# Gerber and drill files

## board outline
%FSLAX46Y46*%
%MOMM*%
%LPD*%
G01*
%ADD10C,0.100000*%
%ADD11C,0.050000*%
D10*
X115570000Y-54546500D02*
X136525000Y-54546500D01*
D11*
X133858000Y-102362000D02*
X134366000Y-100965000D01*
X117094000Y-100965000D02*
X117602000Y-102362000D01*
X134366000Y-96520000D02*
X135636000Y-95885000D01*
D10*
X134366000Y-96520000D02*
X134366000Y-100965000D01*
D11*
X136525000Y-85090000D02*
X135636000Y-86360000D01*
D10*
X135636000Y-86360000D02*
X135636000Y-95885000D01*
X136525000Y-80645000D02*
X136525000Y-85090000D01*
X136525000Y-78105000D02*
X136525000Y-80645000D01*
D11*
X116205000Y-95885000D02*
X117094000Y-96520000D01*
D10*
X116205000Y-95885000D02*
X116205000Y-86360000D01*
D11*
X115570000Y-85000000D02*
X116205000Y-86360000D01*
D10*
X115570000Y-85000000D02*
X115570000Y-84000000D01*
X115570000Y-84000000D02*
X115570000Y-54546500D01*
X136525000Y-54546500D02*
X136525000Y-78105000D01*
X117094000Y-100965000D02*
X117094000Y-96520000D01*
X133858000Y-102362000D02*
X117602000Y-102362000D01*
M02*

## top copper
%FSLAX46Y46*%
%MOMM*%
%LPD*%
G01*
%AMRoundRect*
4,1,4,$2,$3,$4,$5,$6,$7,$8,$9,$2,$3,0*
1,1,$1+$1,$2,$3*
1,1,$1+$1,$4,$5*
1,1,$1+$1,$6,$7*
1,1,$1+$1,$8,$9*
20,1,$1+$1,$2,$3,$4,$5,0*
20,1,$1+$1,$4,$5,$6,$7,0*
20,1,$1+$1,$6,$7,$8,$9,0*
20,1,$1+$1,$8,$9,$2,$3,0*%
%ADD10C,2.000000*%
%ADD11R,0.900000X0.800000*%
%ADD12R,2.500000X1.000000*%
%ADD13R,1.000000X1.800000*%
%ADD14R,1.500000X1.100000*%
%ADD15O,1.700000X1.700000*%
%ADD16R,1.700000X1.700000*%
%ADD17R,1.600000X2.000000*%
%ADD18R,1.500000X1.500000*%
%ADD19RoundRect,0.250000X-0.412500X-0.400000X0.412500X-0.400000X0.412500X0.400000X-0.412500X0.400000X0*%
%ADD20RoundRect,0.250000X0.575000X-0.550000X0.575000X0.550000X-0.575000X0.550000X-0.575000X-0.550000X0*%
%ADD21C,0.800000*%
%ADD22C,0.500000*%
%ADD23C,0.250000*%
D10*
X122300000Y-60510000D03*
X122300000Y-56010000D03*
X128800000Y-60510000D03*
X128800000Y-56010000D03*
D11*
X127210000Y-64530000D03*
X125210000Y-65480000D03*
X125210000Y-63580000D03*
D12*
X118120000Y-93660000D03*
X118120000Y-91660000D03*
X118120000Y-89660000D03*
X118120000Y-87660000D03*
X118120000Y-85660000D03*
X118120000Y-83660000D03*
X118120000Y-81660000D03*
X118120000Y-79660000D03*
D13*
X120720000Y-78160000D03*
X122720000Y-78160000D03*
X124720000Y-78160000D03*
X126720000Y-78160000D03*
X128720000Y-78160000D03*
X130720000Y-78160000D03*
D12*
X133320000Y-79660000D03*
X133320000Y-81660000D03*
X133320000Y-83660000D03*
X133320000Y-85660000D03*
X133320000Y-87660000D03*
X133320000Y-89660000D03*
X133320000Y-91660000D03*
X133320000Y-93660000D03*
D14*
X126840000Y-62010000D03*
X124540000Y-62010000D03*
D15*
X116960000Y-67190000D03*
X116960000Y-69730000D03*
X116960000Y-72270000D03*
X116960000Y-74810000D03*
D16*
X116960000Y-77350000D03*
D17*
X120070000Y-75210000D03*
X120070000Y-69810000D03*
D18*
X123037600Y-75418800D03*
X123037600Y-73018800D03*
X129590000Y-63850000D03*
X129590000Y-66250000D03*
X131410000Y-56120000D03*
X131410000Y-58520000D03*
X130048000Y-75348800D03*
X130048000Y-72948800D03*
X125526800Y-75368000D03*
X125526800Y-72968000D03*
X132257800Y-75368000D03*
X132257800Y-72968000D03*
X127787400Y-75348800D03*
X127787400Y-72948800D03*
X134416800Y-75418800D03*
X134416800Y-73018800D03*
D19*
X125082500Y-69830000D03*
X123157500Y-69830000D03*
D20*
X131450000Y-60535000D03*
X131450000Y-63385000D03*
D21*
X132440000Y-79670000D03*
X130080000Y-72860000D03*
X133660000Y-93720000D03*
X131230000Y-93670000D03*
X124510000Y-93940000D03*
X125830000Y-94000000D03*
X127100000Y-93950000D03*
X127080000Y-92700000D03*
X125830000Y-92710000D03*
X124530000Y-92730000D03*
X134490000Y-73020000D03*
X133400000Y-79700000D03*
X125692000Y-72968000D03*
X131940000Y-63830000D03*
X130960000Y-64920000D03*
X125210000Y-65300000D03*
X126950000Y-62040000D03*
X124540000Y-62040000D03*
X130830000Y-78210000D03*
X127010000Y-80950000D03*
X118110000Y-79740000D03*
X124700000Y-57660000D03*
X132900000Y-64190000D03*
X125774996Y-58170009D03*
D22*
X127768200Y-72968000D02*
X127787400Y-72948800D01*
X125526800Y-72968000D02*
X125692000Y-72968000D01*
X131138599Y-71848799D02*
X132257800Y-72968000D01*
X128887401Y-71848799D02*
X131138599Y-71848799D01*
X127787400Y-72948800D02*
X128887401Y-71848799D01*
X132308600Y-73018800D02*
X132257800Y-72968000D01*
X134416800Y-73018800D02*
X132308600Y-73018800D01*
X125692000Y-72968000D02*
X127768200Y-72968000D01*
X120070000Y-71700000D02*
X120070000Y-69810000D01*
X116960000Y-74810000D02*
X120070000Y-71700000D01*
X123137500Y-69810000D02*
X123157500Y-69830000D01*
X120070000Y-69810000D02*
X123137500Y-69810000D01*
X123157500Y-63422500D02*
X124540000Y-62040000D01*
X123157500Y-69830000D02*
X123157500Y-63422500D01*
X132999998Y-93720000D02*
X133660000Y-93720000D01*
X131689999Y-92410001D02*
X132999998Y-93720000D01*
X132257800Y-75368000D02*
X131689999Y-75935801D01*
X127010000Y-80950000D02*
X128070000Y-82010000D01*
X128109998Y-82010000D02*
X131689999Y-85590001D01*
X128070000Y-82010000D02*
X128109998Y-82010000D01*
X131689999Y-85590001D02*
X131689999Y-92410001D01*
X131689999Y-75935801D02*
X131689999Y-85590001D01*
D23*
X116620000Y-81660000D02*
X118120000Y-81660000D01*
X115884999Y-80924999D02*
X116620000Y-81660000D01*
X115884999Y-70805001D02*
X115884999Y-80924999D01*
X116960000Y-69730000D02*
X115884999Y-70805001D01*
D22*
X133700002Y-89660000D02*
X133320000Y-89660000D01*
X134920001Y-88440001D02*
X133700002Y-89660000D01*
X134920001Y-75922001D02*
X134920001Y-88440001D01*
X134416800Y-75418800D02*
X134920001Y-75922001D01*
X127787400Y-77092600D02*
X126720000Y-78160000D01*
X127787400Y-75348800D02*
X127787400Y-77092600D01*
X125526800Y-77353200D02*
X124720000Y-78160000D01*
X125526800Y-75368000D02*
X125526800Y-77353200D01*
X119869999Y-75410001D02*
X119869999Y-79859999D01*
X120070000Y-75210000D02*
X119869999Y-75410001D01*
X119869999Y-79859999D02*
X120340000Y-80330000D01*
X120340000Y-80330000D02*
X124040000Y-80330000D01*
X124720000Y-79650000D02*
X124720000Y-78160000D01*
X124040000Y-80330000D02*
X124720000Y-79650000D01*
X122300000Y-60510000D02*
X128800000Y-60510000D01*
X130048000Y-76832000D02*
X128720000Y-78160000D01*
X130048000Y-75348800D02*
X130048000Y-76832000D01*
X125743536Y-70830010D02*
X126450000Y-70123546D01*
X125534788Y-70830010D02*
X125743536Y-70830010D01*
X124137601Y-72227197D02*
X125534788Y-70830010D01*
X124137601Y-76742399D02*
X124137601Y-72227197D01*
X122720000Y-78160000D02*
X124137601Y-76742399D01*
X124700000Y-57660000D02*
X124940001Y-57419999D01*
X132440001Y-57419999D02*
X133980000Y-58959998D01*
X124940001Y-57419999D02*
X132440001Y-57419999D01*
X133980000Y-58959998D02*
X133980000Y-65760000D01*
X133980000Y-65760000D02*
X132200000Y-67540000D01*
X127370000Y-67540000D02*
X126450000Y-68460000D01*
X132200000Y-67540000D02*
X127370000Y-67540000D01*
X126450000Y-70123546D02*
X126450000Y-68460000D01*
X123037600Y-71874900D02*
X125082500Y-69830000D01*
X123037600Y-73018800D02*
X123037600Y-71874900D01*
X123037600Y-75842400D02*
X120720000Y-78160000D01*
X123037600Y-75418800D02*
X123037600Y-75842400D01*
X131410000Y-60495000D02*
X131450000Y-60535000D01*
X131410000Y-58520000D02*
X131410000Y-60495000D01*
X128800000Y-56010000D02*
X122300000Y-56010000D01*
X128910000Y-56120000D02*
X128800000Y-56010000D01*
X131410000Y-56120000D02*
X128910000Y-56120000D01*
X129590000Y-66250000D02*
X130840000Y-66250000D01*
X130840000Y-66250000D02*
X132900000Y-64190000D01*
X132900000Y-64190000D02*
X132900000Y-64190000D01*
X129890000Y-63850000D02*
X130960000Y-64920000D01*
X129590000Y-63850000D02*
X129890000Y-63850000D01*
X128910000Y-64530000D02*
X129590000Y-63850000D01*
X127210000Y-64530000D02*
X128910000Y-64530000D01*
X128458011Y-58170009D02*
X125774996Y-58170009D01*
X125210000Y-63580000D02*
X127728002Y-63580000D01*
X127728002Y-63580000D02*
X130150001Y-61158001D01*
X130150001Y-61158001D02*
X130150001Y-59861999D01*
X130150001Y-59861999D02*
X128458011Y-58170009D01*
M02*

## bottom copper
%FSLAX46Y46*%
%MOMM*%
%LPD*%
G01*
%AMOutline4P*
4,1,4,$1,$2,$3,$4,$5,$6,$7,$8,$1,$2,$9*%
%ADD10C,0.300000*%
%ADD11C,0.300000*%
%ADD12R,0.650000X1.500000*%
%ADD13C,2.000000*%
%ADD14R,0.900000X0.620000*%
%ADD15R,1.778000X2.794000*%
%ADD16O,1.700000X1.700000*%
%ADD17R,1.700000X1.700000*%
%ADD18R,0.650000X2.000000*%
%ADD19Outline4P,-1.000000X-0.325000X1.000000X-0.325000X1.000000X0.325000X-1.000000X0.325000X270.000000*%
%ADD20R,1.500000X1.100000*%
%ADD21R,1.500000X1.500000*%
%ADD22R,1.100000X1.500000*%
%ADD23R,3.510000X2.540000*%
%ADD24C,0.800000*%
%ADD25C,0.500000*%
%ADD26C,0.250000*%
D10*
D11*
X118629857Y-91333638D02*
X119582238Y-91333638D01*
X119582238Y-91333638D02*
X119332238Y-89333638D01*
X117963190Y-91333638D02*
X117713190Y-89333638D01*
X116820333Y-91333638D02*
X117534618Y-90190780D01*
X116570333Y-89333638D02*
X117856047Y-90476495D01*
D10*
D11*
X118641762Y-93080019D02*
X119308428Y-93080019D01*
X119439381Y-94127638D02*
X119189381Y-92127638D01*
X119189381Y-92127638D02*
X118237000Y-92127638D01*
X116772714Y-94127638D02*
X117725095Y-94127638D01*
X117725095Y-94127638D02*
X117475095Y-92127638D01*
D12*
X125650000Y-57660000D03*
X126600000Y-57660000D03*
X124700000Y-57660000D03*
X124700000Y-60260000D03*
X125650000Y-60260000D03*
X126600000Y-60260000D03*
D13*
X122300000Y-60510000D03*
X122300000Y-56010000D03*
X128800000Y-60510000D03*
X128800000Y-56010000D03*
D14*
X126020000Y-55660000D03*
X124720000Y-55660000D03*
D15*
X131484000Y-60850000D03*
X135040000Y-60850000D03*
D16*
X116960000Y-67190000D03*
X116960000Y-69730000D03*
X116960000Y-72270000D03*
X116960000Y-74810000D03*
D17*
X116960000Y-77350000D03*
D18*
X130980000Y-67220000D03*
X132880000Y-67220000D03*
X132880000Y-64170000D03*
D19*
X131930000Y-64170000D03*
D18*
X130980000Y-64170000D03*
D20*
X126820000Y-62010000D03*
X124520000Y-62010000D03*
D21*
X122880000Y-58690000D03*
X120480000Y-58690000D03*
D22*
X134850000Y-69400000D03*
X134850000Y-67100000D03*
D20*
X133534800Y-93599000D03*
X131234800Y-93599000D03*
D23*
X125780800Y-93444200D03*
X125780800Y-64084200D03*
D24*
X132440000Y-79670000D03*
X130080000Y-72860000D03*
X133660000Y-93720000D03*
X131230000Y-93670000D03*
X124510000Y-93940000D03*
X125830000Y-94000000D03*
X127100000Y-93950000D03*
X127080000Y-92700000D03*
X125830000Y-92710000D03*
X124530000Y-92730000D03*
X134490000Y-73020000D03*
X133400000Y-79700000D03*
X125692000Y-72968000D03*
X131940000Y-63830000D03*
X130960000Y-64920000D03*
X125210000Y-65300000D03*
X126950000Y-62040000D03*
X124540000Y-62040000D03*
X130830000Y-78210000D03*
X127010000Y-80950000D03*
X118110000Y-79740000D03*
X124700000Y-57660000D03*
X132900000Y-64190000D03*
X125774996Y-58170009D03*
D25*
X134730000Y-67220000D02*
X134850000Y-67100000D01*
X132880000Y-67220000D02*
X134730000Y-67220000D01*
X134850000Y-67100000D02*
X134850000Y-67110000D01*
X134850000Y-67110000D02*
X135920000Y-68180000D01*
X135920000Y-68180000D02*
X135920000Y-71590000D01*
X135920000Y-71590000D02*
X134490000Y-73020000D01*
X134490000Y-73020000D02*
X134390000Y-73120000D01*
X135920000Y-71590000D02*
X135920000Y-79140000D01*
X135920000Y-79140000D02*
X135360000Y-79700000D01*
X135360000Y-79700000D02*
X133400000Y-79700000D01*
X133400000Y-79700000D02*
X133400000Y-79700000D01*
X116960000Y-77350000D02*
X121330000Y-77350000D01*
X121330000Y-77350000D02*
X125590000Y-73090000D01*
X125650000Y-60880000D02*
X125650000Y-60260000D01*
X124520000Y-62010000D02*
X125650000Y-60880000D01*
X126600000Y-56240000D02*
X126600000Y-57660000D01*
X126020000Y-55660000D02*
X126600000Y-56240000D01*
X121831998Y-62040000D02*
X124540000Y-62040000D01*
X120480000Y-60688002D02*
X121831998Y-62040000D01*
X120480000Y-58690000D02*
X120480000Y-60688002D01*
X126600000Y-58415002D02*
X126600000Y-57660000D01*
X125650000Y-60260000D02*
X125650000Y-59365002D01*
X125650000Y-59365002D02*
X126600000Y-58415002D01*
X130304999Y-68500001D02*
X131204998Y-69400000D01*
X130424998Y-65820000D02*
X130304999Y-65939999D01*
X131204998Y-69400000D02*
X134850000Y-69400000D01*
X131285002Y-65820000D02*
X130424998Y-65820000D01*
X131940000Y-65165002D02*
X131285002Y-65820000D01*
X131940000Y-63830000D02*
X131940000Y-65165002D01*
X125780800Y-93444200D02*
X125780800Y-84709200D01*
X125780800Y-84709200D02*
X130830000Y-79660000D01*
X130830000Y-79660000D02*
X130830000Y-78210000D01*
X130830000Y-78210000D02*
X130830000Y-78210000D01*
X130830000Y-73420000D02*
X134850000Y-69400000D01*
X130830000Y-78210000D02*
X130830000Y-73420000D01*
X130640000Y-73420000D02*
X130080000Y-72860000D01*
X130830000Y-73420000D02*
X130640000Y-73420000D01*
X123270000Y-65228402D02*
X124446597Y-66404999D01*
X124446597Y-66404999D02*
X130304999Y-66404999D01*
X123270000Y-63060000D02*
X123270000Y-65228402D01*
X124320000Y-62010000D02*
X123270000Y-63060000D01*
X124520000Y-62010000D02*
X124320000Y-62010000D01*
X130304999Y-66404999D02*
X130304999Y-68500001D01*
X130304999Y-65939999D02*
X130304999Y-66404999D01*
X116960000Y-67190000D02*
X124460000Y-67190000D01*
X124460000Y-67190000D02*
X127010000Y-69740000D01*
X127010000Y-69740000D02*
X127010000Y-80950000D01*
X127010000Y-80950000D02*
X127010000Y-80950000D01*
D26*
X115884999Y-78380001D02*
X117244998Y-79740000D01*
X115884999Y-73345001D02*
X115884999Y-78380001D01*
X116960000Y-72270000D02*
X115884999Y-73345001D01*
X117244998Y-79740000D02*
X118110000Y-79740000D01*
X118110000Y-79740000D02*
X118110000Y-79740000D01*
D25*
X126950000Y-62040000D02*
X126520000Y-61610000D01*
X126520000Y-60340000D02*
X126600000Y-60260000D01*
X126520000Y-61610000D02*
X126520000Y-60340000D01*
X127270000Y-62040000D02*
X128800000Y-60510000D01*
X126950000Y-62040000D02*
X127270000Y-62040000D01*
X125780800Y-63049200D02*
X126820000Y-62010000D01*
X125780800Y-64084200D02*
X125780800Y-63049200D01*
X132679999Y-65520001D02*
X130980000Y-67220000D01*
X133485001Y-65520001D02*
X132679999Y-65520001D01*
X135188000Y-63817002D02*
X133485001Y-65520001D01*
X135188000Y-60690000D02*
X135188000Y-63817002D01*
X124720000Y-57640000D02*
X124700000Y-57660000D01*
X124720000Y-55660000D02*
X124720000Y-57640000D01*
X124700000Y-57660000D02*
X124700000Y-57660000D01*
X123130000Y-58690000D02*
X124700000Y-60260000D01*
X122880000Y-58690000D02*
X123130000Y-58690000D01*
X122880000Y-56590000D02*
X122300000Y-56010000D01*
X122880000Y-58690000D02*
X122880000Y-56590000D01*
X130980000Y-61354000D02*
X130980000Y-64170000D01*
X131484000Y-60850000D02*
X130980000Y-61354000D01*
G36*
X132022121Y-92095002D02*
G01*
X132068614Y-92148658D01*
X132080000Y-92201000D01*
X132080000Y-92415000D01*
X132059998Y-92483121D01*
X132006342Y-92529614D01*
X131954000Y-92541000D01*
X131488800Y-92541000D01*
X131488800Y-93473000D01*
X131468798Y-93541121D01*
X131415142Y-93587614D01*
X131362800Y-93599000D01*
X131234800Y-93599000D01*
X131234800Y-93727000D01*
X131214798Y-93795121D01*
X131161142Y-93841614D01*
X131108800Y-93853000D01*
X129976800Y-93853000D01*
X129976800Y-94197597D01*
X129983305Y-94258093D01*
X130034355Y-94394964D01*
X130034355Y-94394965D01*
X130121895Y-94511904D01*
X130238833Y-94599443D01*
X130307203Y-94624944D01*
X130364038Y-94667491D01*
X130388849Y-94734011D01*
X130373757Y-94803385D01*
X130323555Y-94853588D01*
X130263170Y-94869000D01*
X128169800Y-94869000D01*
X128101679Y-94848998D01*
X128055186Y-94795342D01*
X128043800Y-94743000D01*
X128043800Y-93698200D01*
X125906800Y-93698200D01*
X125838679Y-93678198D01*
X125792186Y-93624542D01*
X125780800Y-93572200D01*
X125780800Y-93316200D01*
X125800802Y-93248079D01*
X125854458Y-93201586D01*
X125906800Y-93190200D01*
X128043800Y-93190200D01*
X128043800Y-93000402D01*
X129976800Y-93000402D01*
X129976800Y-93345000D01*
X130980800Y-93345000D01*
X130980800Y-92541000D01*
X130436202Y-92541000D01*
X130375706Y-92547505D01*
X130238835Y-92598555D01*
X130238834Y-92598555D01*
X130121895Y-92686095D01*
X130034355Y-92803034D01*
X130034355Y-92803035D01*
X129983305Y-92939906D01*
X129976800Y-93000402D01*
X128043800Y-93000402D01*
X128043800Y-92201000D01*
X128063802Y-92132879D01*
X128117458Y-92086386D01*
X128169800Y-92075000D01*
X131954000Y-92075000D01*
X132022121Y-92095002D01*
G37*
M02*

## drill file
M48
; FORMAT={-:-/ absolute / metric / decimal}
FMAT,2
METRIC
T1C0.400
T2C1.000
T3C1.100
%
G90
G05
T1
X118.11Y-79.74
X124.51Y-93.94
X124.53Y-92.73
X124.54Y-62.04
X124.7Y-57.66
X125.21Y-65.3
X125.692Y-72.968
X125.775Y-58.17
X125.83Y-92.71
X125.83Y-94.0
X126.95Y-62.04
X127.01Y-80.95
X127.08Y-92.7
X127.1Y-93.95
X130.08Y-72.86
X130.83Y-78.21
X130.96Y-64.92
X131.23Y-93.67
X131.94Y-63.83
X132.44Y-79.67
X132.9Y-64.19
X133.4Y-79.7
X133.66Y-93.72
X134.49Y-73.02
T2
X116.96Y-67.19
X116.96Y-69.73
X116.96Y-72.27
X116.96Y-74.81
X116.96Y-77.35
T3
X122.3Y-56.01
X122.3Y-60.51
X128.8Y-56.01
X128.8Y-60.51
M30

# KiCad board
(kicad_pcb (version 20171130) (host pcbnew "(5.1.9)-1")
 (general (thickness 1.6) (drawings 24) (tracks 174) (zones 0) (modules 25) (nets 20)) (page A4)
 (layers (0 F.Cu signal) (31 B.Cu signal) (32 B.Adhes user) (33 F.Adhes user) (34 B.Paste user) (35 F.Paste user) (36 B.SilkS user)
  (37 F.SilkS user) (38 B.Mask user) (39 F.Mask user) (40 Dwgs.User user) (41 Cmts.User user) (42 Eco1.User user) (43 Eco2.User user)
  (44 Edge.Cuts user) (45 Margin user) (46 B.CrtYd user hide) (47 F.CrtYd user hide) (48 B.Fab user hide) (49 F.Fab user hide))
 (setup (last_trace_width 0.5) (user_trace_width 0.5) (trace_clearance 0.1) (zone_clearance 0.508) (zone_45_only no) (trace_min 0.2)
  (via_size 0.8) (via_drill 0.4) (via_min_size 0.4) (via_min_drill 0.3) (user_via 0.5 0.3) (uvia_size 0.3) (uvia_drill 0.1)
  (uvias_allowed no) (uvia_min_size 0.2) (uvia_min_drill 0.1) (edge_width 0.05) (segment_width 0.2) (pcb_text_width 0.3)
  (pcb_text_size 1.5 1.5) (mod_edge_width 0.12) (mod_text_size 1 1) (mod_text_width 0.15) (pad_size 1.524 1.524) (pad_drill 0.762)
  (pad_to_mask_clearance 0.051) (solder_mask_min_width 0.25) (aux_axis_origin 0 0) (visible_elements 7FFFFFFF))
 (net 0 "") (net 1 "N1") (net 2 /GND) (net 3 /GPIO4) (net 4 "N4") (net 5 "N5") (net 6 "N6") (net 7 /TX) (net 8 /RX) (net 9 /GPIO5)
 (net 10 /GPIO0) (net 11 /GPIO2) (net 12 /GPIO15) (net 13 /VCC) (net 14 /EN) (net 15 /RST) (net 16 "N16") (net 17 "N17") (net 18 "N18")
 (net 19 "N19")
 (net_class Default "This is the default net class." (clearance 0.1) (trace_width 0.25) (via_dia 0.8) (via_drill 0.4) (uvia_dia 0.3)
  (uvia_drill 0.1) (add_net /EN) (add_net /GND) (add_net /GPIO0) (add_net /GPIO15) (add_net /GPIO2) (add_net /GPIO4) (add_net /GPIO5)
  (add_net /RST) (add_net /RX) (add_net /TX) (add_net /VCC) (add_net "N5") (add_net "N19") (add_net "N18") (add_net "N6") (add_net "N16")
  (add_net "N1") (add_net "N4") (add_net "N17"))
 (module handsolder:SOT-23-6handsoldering (layer B.Cu) (at 125.65 58.96 90)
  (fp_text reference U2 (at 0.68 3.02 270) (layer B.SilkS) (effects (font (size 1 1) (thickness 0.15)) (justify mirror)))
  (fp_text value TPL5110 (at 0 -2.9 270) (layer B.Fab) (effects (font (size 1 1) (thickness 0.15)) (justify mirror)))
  (pad 5 smd rect (at 1.3 0 90) (size 1.5 0.65) (layers B.Cu B.Paste B.Mask) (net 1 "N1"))
  (pad 6 smd rect (at 1.3 0.95 90) (size 1.5 0.65) (layers B.Cu B.Paste B.Mask) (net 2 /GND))
  (pad 4 smd rect (at 1.3 -0.95 90) (size 1.5 0.65) (layers B.Cu B.Paste B.Mask) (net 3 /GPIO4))
  (pad 3 smd rect (at -1.3 -0.95 90) (size 1.5 0.65) (layers B.Cu B.Paste B.Mask) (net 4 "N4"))
  (pad 2 smd rect (at -1.3 0 90) (size 1.5 0.65) (layers B.Cu B.Paste B.Mask) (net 2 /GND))
  (pad 1 smd rect (at -1.3 0.95 90) (size 1.5 0.65) (layers B.Cu B.Paste B.Mask) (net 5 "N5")))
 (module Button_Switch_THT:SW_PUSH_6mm (layer F.Cu) (at 128.8 60.51 180)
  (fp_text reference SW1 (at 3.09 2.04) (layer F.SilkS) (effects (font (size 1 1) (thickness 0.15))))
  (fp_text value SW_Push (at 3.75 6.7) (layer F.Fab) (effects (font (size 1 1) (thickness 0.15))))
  (pad 1 thru_hole circle (at 6.5 0 270) (size 2 2) (drill 1.1) (layers *.Cu *.Mask) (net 5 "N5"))
  (pad 2 thru_hole circle (at 6.5 4.5 270) (size 2 2) (drill 1.1) (layers *.Cu *.Mask) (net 4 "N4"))
  (pad 1 thru_hole circle (at 0 0 270) (size 2 2) (drill 1.1) (layers *.Cu *.Mask) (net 5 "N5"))
  (pad 2 thru_hole circle (at 0 4.5 270) (size 2 2) (drill 1.1) (layers *.Cu *.Mask) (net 4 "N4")))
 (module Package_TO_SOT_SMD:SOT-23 (layer F.Cu) (at 126.21 64.53)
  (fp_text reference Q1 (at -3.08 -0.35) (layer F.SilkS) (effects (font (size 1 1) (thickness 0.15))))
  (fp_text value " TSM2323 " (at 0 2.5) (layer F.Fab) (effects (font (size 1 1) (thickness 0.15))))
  (pad 3 smd rect (at 1 0) (size 0.9 0.8) (layers F.Cu F.Paste F.Mask) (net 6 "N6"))
  (pad 2 smd rect (at -1 0.95) (size 0.9 0.8) (layers F.Cu F.Paste F.Mask) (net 5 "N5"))
  (pad 1 smd rect (at -1 -0.95) (size 0.9 0.8) (layers F.Cu F.Paste F.Mask) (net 1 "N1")))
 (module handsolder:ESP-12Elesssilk (layer F.Cu) (at 125.72 90.16 180)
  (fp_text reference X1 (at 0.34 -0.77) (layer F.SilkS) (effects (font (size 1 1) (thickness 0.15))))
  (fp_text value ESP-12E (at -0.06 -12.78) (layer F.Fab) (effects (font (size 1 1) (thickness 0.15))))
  (pad 22 smd rect (at 7.6 -3.5 180) (size 2.5 1) (layers F.Cu F.Paste F.Mask))
  (pad 21 smd rect (at 7.6 -1.5 180) (size 2.5 1) (layers F.Cu F.Paste F.Mask))
  (pad 20 smd rect (at 7.6 0.5 180) (size 2.5 1) (layers F.Cu F.Paste F.Mask))
  (pad 19 smd rect (at 7.6 2.5 180) (size 2.5 1) (layers F.Cu F.Paste F.Mask))
  (pad 18 smd rect (at 7.6 4.5 180) (size 2.5 1) (layers F.Cu F.Paste F.Mask))
  (pad 17 smd rect (at 7.6 6.5 180) (size 2.5 1) (layers F.Cu F.Paste F.Mask))
  (pad 16 smd rect (at 7.6 8.5 180) (size 2.5 1) (layers F.Cu F.Paste F.Mask) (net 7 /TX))
  (pad 15 smd rect (at 7.6 10.5 180) (size 2.5 1) (layers F.Cu F.Paste F.Mask) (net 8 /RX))
  (pad 14 smd rect (at 5 12 180) (size 1 1.8) (layers F.Cu F.Paste F.Mask) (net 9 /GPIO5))
  (pad 13 smd rect (at 3 12 180) (size 1 1.8) (layers F.Cu F.Paste F.Mask) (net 3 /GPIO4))
  (pad 12 smd rect (at 1 12 180) (size 1 1.8) (layers F.Cu F.Paste F.Mask) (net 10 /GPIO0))
  (pad 11 smd rect (at -1 12 180) (size 1 1.8) (layers F.Cu F.Paste F.Mask) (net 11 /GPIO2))
  (pad 10 smd rect (at -3 12 180) (size 1 1.8) (layers F.Cu F.Paste F.Mask) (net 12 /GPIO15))
  (pad 9 smd rect (at -5 12 180) (size 1 1.8) (layers F.Cu F.Paste F.Mask) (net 2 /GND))
  (pad 8 smd rect (at -7.6 10.5 180) (size 2.5 1) (layers F.Cu F.Paste F.Mask) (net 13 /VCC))
  (pad 7 smd rect (at -7.6 8.5 180) (size 2.5 1) (layers F.Cu F.Paste F.Mask))
  (pad 6 smd rect (at -7.6 6.5 180) (size 2.5 1) (layers F.Cu F.Paste F.Mask))
  (pad 5 smd rect (at -7.6 4.5 180) (size 2.5 1) (layers F.Cu F.Paste F.Mask))
  (pad 4 smd rect (at -7.6 2.5 180) (size 2.5 1) (layers F.Cu F.Paste F.Mask))
  (pad 3 smd rect (at -7.6 0.5 180) (size 2.5 1) (layers F.Cu F.Paste F.Mask) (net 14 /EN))
  (pad 2 smd rect (at -7.6 -1.5 180) (size 2.5 1) (layers F.Cu F.Paste F.Mask))
  (pad 1 smd rect (at -7.6 -3.5 180) (size 2.5 1) (layers F.Cu F.Paste F.Mask) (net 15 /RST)))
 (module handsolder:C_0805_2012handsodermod (layer F.Cu) (at 125.69 62.01)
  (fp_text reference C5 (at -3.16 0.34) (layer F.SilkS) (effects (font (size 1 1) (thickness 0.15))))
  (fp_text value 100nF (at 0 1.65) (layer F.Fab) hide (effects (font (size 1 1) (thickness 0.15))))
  (pad 2 smd rect (at 1.15 0) (size 1.5 1.1) (layers F.Cu F.Paste F.Mask) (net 5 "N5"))
  (pad 1 smd rect (at -1.15 0) (size 1.5 1.1) (layers F.Cu F.Paste F.Mask) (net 2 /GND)))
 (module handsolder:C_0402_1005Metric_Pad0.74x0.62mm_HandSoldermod (layer B.Cu) (at 125.37 55.66)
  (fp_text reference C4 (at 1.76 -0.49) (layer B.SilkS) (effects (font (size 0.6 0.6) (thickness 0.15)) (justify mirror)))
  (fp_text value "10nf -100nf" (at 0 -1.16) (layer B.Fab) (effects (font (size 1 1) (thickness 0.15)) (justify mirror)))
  (pad 2 smd rect (at 0.65 0) (size 0.9 0.62) (layers B.Cu B.Paste B.Mask) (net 2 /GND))
  (pad 1 smd rect (at -0.65 0) (size 0.9 0.62) (layers B.Cu B.Paste B.Mask) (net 3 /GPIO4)))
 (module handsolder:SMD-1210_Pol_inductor (layer B.Cu) (at 133.262 60.85)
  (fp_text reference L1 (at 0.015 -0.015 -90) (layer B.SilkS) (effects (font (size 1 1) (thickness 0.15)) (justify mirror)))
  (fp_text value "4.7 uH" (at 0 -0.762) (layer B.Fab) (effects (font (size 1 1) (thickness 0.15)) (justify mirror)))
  (pad 1 smd rect (at -1.778 0) (size 1.778 2.794) (layers B.Cu B.Paste B.Mask) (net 6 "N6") (zone_connect 2))
  (pad 2 smd rect (at 1.778 0) (size 1.778 2.794) (layers B.Cu B.Paste B.Mask) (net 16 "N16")))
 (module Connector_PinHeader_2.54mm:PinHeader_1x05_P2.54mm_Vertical (layer F.Cu) (at 116.96 77.35 180)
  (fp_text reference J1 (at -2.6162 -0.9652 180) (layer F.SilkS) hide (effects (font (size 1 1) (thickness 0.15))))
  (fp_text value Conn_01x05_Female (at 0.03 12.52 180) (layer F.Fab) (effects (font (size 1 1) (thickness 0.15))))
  (pad 5 thru_hole oval (at 0 10.16 180) (size 1.7 1.7) (drill 1) (layers *.Cu *.Mask) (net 15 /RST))
  (pad 4 thru_hole oval (at 0 7.62 180) (size 1.7 1.7) (drill 1) (layers *.Cu *.Mask) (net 7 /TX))
  (pad 3 thru_hole oval (at 0 5.08 180) (size 1.7 1.7) (drill 1) (layers *.Cu *.Mask) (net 8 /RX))
  (pad 2 thru_hole oval (at 0 2.54 180) (size 1.7 1.7) (drill 1) (layers *.Cu *.Mask) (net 2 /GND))
  (pad 1 thru_hole rect (at 0 0 180) (size 1.7 1.7) (drill 1) (layers *.Cu *.Mask) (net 13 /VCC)))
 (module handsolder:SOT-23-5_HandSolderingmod (layer B.Cu) (at 131.93 65.72 270)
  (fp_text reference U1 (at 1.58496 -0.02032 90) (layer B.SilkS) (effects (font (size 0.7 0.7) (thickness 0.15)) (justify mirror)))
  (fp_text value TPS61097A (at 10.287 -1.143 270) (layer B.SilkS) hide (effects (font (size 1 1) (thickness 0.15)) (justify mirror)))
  (pad 5 smd rect (at 1.5 0.95 270) (size 2 0.65) (layers B.Cu B.Paste B.Mask) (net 16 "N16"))
  (pad 4 smd rect (at 1.5 -0.95 270) (size 2 0.65) (layers B.Cu B.Paste B.Mask) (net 13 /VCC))
  (pad 3 smd rect (at -1.55 -0.95 270) (size 2 0.65) (layers B.Cu B.Paste B.Mask) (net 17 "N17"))
  (pad 2 smd trapezoid (at -1.55 0 270) (size 2 0.65) (layers B.Cu B.Paste B.Mask) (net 2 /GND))
  (pad 1 smd rect (at -1.55 0.95 270) (size 2 0.65) (layers B.Cu B.Paste B.Mask) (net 6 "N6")))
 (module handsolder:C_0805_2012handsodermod (layer B.Cu) (at 125.67 62.01)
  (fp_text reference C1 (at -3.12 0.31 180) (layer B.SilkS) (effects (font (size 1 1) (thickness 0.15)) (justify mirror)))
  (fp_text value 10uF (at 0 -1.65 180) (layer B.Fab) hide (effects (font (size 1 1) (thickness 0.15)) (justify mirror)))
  (pad 2 smd rect (at 1.15 0) (size 1.5 1.1) (layers B.Cu B.Paste B.Mask) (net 5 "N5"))
  (pad 1 smd rect (at -1.15 0) (size 1.5 1.1) (layers B.Cu B.Paste B.Mask) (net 2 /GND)))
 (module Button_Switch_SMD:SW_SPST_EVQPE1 (layer F.Cu) (at 120.07 72.51 90)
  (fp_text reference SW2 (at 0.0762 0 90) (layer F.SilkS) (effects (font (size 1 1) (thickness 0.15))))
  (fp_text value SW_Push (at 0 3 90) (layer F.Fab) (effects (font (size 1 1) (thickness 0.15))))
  (pad 1 smd rect (at -2.7 0 90) (size 2 1.6) (layers F.Cu F.Paste F.Mask) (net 10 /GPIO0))
  (pad 2 smd rect (at 2.7 0 90) (size 2 1.6) (layers F.Cu F.Paste F.Mask) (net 2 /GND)))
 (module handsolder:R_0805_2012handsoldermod (layer F.Cu) (at 123.0376 74.2188 270)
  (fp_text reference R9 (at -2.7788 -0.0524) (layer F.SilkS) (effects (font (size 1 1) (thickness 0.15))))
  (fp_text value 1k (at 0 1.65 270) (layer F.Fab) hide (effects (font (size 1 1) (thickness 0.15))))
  (pad 2 smd rect (at 1.2 0 270) (size 1.5 1.5) (layers F.Cu F.Paste F.Mask) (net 9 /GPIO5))
  (pad 1 smd rect (at -1.2 0 270) (size 1.5 1.5) (layers F.Cu F.Paste F.Mask) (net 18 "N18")))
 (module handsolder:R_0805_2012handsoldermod (layer B.Cu) (at 121.68 58.69)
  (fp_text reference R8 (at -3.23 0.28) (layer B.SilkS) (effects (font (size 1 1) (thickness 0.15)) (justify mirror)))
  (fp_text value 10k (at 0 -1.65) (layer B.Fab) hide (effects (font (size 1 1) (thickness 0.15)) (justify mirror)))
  (pad 2 smd rect (at 1.2 0) (size 1.5 1.5) (layers B.Cu B.Paste B.Mask) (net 4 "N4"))
  (pad 1 smd rect (at -1.2 0) (size 1.5 1.5) (layers B.Cu B.Paste B.Mask) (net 2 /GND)))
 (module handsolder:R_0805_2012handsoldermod (layer F.Cu) (at 129.59 65.05 90)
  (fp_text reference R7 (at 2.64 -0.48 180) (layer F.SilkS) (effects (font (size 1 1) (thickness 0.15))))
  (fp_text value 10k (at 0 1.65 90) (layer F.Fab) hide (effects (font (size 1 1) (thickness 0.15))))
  (pad 2 smd rect (at 1.2 0 90) (size 1.5 1.5) (layers F.Cu F.Paste F.Mask) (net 6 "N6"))
  (pad 1 smd rect (at -1.2 0 90) (size 1.5 1.5) (layers F.Cu F.Paste F.Mask) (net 17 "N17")))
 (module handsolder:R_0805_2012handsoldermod (layer F.Cu) (at 131.41 57.32 90)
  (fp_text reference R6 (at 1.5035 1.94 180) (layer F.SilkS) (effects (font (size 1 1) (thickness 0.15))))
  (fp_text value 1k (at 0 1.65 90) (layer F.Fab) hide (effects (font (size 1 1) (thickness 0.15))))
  (pad 2 smd rect (at 1.2 0 90) (size 1.5 1.5) (layers F.Cu F.Paste F.Mask) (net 4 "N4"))
  (pad 1 smd rect (at -1.2 0 90) (size 1.5 1.5) (layers F.Cu F.Paste F.Mask) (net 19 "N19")))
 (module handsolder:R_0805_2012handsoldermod (layer F.Cu) (at 130.048 74.1488 270)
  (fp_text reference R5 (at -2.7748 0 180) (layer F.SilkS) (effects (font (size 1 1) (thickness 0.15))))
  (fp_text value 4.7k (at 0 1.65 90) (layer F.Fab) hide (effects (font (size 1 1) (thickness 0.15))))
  (pad 2 smd rect (at 1.2 0 270) (size 1.5 1.5) (layers F.Cu F.Paste F.Mask) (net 12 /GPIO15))
  (pad 1 smd rect (at -1.2 0 270) (size 1.5 1.5) (layers F.Cu F.Paste F.Mask) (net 2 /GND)))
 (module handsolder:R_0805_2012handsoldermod (layer F.Cu) (at 125.5268 74.168 270)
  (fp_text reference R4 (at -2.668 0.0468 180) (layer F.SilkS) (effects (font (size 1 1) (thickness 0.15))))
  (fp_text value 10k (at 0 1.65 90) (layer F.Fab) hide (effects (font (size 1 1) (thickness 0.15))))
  (pad 2 smd rect (at 1.2 0 270) (size 1.5 1.5) (layers F.Cu F.Paste F.Mask) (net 10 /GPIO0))
  (pad 1 smd rect (at -1.2 0 270) (size 1.5 1.5) (layers F.Cu F.Paste F.Mask) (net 13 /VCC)))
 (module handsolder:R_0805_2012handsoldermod (layer F.Cu) (at 132.2578 74.168 270)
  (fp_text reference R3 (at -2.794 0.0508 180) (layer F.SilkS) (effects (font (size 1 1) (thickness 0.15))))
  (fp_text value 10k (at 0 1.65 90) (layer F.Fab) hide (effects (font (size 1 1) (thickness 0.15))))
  (pad 2 smd rect (at 1.2 0 270) (size 1.5 1.5) (layers F.Cu F.Paste F.Mask) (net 15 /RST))
  (pad 1 smd rect (at -1.2 0 270) (size 1.5 1.5) (layers F.Cu F.Paste F.Mask) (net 13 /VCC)))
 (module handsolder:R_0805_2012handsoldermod (layer F.Cu) (at 127.7874 74.1488 270)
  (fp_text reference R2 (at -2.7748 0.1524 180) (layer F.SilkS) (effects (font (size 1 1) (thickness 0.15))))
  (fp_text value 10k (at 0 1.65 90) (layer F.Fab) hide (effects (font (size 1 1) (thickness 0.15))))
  (pad 2 smd rect (at 1.2 0 270) (size 1.5 1.5) (layers F.Cu F.Paste F.Mask) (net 11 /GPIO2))
  (pad 1 smd rect (at -1.2 0 270) (size 1.5 1.5) (layers F.Cu F.Paste F.Mask) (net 13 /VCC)))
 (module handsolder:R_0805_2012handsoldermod (layer F.Cu) (at 134.4168 74.2188 270)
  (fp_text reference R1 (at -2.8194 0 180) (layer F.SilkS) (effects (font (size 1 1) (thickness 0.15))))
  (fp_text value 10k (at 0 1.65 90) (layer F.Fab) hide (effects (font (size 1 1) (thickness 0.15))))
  (pad 2 smd rect (at 1.2 0 270) (size 1.5 1.5) (layers F.Cu F.Paste F.Mask) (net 14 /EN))
  (pad 1 smd rect (at -1.2 0 270) (size 1.5 1.5) (layers F.Cu F.Paste F.Mask) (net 13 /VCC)))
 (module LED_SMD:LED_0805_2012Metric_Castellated (layer F.Cu) (at 124.12 69.83)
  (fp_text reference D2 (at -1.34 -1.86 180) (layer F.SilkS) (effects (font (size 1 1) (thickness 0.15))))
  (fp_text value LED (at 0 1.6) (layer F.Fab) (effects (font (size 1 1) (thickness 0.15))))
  (pad 2 smd roundrect (at 0.9625 0) (size 1.325 1.3) (layers F.Cu F.Paste F.Mask) (roundrect_rratio 0.1923076923076923) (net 18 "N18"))
  (pad 1 smd roundrect (at -0.9625 0) (size 1.325 1.3) (layers F.Cu F.Paste F.Mask) (roundrect_rratio 0.1923076923076923) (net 2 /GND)))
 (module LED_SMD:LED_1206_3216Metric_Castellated (layer F.Cu) (at 131.45 61.96 90)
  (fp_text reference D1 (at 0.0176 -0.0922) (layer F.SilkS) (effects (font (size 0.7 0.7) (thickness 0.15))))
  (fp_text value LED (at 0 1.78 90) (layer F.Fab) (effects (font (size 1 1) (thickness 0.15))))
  (pad 2 smd roundrect (at 1.425 0 90) (size 1.6 1.65) (layers F.Cu F.Paste F.Mask) (roundrect_rratio 0.15625) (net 19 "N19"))
  (pad 1 smd roundrect (at -1.425 0 90) (size 1.6 1.65) (layers F.Cu F.Paste F.Mask) (roundrect_rratio 0.15625) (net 2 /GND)))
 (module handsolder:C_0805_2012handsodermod (layer B.Cu) (at 134.85 68.25 270)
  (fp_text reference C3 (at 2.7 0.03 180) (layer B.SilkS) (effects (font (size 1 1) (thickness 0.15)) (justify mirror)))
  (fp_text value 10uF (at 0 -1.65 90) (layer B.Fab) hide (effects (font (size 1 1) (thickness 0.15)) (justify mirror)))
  (pad 2 smd rect (at 1.15 0 270) (size 1.5 1.1) (layers B.Cu B.Paste B.Mask) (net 2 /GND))
  (pad 1 smd rect (at -1.15 0 270) (size 1.5 1.1) (layers B.Cu B.Paste B.Mask) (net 13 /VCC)))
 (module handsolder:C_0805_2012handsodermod (layer B.Cu) (at 132.3848 93.599)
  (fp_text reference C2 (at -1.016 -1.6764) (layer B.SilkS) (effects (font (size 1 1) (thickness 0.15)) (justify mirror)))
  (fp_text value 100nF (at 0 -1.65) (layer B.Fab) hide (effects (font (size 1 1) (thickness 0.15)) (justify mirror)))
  (pad 2 smd rect (at 1.15 0) (size 1.5 1.1) (layers B.Cu B.Paste B.Mask) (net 15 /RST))
  (pad 1 smd rect (at -1.15 0) (size 1.5 1.1) (layers B.Cu B.Paste B.Mask) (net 2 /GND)))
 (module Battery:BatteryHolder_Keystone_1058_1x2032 (layer B.Cu) (at 125.7808 78.7642 270)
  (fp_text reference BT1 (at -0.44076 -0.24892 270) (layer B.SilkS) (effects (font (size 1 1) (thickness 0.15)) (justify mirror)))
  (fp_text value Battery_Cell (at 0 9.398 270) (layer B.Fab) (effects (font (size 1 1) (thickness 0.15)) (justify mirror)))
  (pad 2 smd rect (at 14.68 0 270) (size 2.54 3.51) (layers B.Cu B.Paste B.Mask) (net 2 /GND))
  (pad 1 smd rect (at -14.68 0 270) (size 2.54 3.51) (layers B.Cu B.Paste B.Mask) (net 5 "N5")))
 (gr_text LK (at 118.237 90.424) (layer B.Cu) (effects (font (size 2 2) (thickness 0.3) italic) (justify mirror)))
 (gr_line (start 115.57 54.5465) (end 136.525 54.5465) (layer Edge.Cuts) (width 0.1))
 (gr_line (start 133.858 102.362) (end 134.366 100.965) (layer Edge.Cuts) (width 0.05))
 (gr_line (start 117.094 100.965) (end 117.602 102.362) (layer Edge.Cuts) (width 0.05))
 (gr_line (start 134.366 96.52) (end 135.636 95.885) (layer Edge.Cuts) (width 0.05))
 (gr_line (start 134.366 96.52) (end 134.366 100.965) (layer Edge.Cuts) (width 0.1))
 (gr_line (start 136.525 85.09) (end 135.636 86.36) (layer Edge.Cuts) (width 0.05))
 (gr_line (start 135.636 86.36) (end 135.636 95.885) (layer Edge.Cuts) (width 0.1))
 (gr_line (start 136.525 80.645) (end 136.525 85.09) (layer Edge.Cuts) (width 0.1))
 (gr_line (start 136.525 78.105) (end 136.525 80.645) (layer Edge.Cuts) (width 0.1))
 (gr_line (start 116.205 95.885) (end 117.094 96.52) (layer Edge.Cuts) (width 0.05))
 (gr_line (start 116.205 95.885) (end 116.205 86.36) (layer Edge.Cuts) (width 0.1))
 (gr_line (start 115.57 85) (end 116.205 86.36) (layer Edge.Cuts) (width 0.05))
 (gr_line (start 115.57 85) (end 115.57 84) (layer Edge.Cuts) (width 0.1))
 (gr_line (start 115.57 84) (end 115.57 54.5465) (layer Edge.Cuts) (width 0.1))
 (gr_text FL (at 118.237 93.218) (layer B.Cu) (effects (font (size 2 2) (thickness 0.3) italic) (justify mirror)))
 (gr_line (start 136.525 54.5465) (end 136.525 78.105) (layer Edge.Cuts) (width 0.1))
 (gr_line (start 117.094 100.965) (end 117.094 96.52) (layer Edge.Cuts) (width 0.1))
 (gr_line (start 133.858 102.362) (end 117.602 102.362) (layer Edge.Cuts) (width 0.1))
 (via (at 132.44 79.67) (size 0.8) (drill 0.4) (layers F.Cu B.Cu) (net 13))
 (via (at 130.08 72.86) (size 0.8) (drill 0.4) (layers F.Cu B.Cu) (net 2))
 (via (at 133.66 93.72) (size 0.8) (drill 0.4) (layers F.Cu B.Cu) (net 15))
 (via (at 131.23 93.67) (size 0.8) (drill 0.4) (layers F.Cu B.Cu) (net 2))
 (via (at 124.51 93.94) (size 0.8) (drill 0.4) (layers F.Cu B.Cu) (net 2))
 (via (at 125.83 94) (size 0.8) (drill 0.4) (layers F.Cu B.Cu) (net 2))
 (via (at 127.1 93.95) (size 0.8) (drill 0.4) (layers F.Cu B.Cu) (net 2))
 (via (at 127.08 92.7) (size 0.8) (drill 0.4) (layers F.Cu B.Cu) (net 2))
 (via (at 125.83 92.71) (size 0.8) (drill 0.4) (layers F.Cu B.Cu) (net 2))
 (via (at 124.53 92.73) (size 0.8) (drill 0.4) (layers F.Cu B.Cu) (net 2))
 (segment (start 134.73 67.22) (end 134.85 67.1) (width 0.5) (layer B.Cu) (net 13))
 (segment (start 132.88 67.22) (end 134.73 67.22) (width 0.5) (layer B.Cu) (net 13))
 (segment (start 127.7682 72.968) (end 127.7874 72.9488) (width 0.5) (layer F.Cu) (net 13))
 (segment (start 125.5268 72.968) (end 125.692 72.968) (width 0.5) (layer F.Cu) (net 13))
 (segment (start 131.138599 71.848799) (end 132.2578 72.968) (width 0.5) (layer F.Cu) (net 13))
 (segment (start 128.887401 71.848799) (end 131.138599 71.848799) (width 0.5) (layer F.Cu) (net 13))
 (segment (start 127.7874 72.9488) (end 128.887401 71.848799) (width 0.5) (layer F.Cu) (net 13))
 (segment (start 132.3086 73.0188) (end 132.2578 72.968) (width 0.5) (layer F.Cu) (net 13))
 (segment (start 134.4168 73.0188) (end 132.3086 73.0188) (width 0.5) (layer F.Cu) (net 13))
 (segment (start 134.85 67.1) (end 134.85 67.11) (width 0.5) (layer B.Cu) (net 13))
 (segment (start 134.85 67.11) (end 135.92 68.18) (width 0.5) (layer B.Cu) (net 13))
 (segment (start 135.92 68.18) (end 135.92 71.59) (width 0.5) (layer B.Cu) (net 13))
 (segment (start 135.92 71.59) (end 134.49 73.02) (width 0.5) (layer B.Cu) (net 13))
 (segment (start 134.49 73.02) (end 134.39 73.12) (width 0.5) (layer B.Cu) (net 13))
 (via (at 134.49 73.02) (size 0.8) (drill 0.4) (layers F.Cu B.Cu) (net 13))
 (segment (start 135.92 71.59) (end 135.92 79.14) (width 0.5) (layer B.Cu) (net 13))
 (segment (start 135.92 79.14) (end 135.36 79.7) (width 0.5) (layer B.Cu) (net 13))
 (segment (start 135.36 79.7) (end 133.4 79.7) (width 0.5) (layer B.Cu) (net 13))
 (segment (start 133.4 79.7) (end 133.4 79.7) (width 0.5) (layer B.Cu) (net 13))
 (via (at 133.4 79.7) (size 0.8) (drill 0.4) (layers F.Cu B.Cu) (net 13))
 (segment (start 116.96 77.35) (end 121.33 77.35) (width 0.5) (layer B.Cu) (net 13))
 (segment (start 121.33 77.35) (end 125.59 73.09) (width 0.5) (layer B.Cu) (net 13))
 (segment (start 125.692 72.968) (end 127.7682 72.968) (width 0.5) (layer F.Cu) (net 13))
 (via (at 125.692 72.968) (size 0.8) (drill 0.4) (layers F.Cu B.Cu) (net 13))
 (via (at 131.94 63.83) (size 0.8) (drill 0.4) (layers F.Cu B.Cu) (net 2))
 (via (at 130.96 64.92) (size 0.8) (drill 0.4) (layers F.Cu B.Cu) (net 6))
 (via (at 125.21 65.3) (size 0.8) (drill 0.4) (layers F.Cu B.Cu) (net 5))
 (via (at 126.95 62.04) (size 0.8) (drill 0.4) (layers F.Cu B.Cu) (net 5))
 (via (at 124.54 62.04) (size 0.8) (drill 0.4) (layers F.Cu B.Cu) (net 2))
 (segment (start 125.65 60.88) (end 125.65 60.26) (width 0.5) (layer B.Cu) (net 2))
 (segment (start 124.52 62.01) (end 125.65 60.88) (width 0.5) (layer B.Cu) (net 2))
 (segment (start 126.6 56.24) (end 126.6 57.66) (width 0.5) (layer B.Cu) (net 2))
 (segment (start 126.02 55.66) (end 126.6 56.24) (width 0.5) (layer B.Cu) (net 2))
 (segment (start 121.831998 62.04) (end 124.54 62.04) (width 0.5) (layer B.Cu) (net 2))
 (segment (start 120.48 60.688002) (end 121.831998 62.04) (width 0.5) (layer B.Cu) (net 2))
 (segment (start 120.48 58.69) (end 120.48 60.688002) (width 0.5) (layer B.Cu) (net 2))
 (segment (start 126.6 58.415002) (end 126.6 57.66) (width 0.5) (layer B.Cu) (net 2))
 (segment (start 125.65 60.26) (end 125.65 59.365002) (width 0.5) (layer B.Cu) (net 2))
 (segment (start 125.65 59.365002) (end 126.6 58.415002) (width 0.5) (layer B.Cu) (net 2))
 (segment (start 130.304999 68.500001) (end 131.204998 69.4) (width 0.5) (layer B.Cu) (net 2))
 (segment (start 130.424998 65.82) (end 130.304999 65.939999) (width 0.5) (layer B.Cu) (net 2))
 (segment (start 131.204998 69.4) (end 134.85 69.4) (width 0.5) (layer B.Cu) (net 2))
 (segment (start 131.285002 65.82) (end 130.424998 65.82) (width 0.5) (layer B.Cu) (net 2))
 (segment (start 131.94 65.165002) (end 131.285002 65.82) (width 0.5) (layer B.Cu) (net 2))
 (segment (start 131.94 63.83) (end 131.94 65.165002) (width 0.5) (layer B.Cu) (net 2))
 (segment (start 125.7808 93.4442) (end 125.7808 84.7092) (width 0.5) (layer B.Cu) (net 2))
 (segment (start 125.7808 84.7092) (end 130.83 79.66) (width 0.5) (layer B.Cu) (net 2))
 (segment (start 130.83 79.66) (end 130.83 78.21) (width 0.5) (layer B.Cu) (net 2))
 (segment (start 130.83 78.21) (end 130.83 78.21) (width 0.5) (layer B.Cu) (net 2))
 (via (at 130.83 78.21) (size 0.8) (drill 0.4) (layers F.Cu B.Cu) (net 2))
 (segment (start 130.83 73.42) (end 134.85 69.4) (width 0.5) (layer B.Cu) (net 2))
 (segment (start 130.83 78.21) (end 130.83 73.42) (width 0.5) (layer B.Cu) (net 2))
 (segment (start 130.64 73.42) (end 130.08 72.86) (width 0.5) (layer B.Cu) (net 2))
 (segment (start 130.83 73.42) (end 130.64 73.42) (width 0.5) (layer B.Cu) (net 2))
 (segment (start 120.07 71.7) (end 120.07 69.81) (width 0.5) (layer F.Cu) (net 2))
 (segment (start 116.96 74.81) (end 120.07 71.7) (width 0.5) (layer F.Cu) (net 2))
 (segment (start 123.1375 69.81) (end 123.1575 69.83) (width 0.5) (layer F.Cu) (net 2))
 (segment (start 120.07 69.81) (end 123.1375 69.81) (width 0.5) (layer F.Cu) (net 2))
 (segment (start 123.1575 63.4225) (end 124.54 62.04) (width 0.5) (layer F.Cu) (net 2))
 (segment (start 123.1575 69.83) (end 123.1575 63.4225) (width 0.5) (layer F.Cu) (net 2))
 (segment (start 123.27 65.228402) (end 124.446597 66.404999) (width 0.5) (layer B.Cu) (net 2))
 (segment (start 124.446597 66.404999) (end 130.304999 66.404999) (width 0.5) (layer B.Cu) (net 2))
 (segment (start 123.27 63.06) (end 123.27 65.228402) (width 0.5) (layer B.Cu) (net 2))
 (segment (start 124.32 62.01) (end 123.27 63.06) (width 0.5) (layer B.Cu) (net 2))
 (segment (start 124.52 62.01) (end 124.32 62.01) (width 0.5) (layer B.Cu) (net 2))
 (segment (start 130.304999 66.404999) (end 130.304999 68.500001) (width 0.5) (layer B.Cu) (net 2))
 (segment (start 130.304999 65.939999) (end 130.304999 66.404999) (width 0.5) (layer B.Cu) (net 2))
 (segment (start 132.999998 93.72) (end 133.66 93.72) (width 0.5) (layer F.Cu) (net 15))
 (segment (start 131.689999 92.410001) (end 132.999998 93.72) (width 0.5) (layer F.Cu) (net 15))
 (segment (start 132.2578 75.368) (end 131.689999 75.935801) (width 0.5) (layer F.Cu) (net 15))
 (segment (start 116.96 67.19) (end 124.46 67.19) (width 0.5) (layer B.Cu) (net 15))
 (segment (start 124.46 67.19) (end 127.01 69.74) (width 0.5) (layer B.Cu) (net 15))
 (segment (start 127.01 69.74) (end 127.01 80.95) (width 0.5) (layer B.Cu) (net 15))
 (segment (start 127.01 80.95) (end 127.01 80.95) (width 0.5) (layer B.Cu) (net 15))
 (via (at 127.01 80.95) (size 0.8) (drill 0.4) (layers F.Cu B.Cu) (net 15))
 (segment (start 127.01 80.95) (end 128.07 82.01) (width 0.5) (layer F.Cu) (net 15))
 (segment (start 128.109998 82.01) (end 131.689999 85.590001) (width 0.5) (layer F.Cu) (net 15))
 (segment (start 128.07 82.01) (end 128.109998 82.01) (width 0.5) (layer F.Cu) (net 15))
 (segment (start 131.689999 85.590001) (end 131.689999 92.410001) (width 0.5) (layer F.Cu) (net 15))
 (segment (start 131.689999 75.935801) (end 131.689999 85.590001) (width 0.5) (layer F.Cu) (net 15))
 (segment (start 115.884999 78.380001) (end 117.244998 79.74) (width 0.25) (layer B.Cu) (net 8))
 (segment (start 115.884999 73.345001) (end 115.884999 78.380001) (width 0.25) (layer B.Cu) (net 8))
 (segment (start 116.96 72.27) (end 115.884999 73.345001) (width 0.25) (layer B.Cu) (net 8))
 (segment (start 117.244998 79.74) (end 118.11 79.74) (width 0.25) (layer B.Cu) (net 8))
 (segment (start 118.11 79.74) (end 118.11 79.74) (width 0.25) (layer B.Cu) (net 8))
 (via (at 118.11 79.74) (size 0.8) (drill 0.4) (layers F.Cu B.Cu) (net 8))
 (segment (start 116.62 81.66) (end 118.12 81.66) (width 0.25) (layer F.Cu) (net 7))
 (segment (start 115.884999 80.924999) (end 116.62 81.66) (width 0.25) (layer F.Cu) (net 7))
 (segment (start 115.884999 70.805001) (end 115.884999 80.924999) (width 0.25) (layer F.Cu) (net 7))
 (segment (start 116.96 69.73) (end 115.884999 70.805001) (width 0.25) (layer F.Cu) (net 7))
 (segment (start 133.700002 89.66) (end 133.32 89.66) (width 0.5) (layer F.Cu) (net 14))
 (segment (start 134.920001 88.440001) (end 133.700002 89.66) (width 0.5) (layer F.Cu) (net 14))
 (segment (start 134.920001 75.922001) (end 134.920001 88.440001) (width 0.5) (layer F.Cu) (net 14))
 (segment (start 134.4168 75.4188) (end 134.920001 75.922001) (width 0.5) (layer F.Cu) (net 14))
 (segment (start 127.7874 77.0926) (end 126.72 78.16) (width 0.5) (layer F.Cu) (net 11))
 (segment (start 127.7874 75.3488) (end 127.7874 77.0926) (width 0.5) (layer F.Cu) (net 11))
 (segment (start 125.5268 77.3532) (end 124.72 78.16) (width 0.5) (layer F.Cu) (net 10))
 (segment (start 125.5268 75.368) (end 125.5268 77.3532) (width 0.5) (layer F.Cu) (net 10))
 (segment (start 119.869999 75.410001) (end 119.869999 79.859999) (width 0.5) (layer F.Cu) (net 10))
 (segment (start 120.07 75.21) (end 119.869999 75.410001) (width 0.5) (layer F.Cu) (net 10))
 (segment (start 119.869999 79.859999) (end 120.34 80.33) (width 0.5) (layer F.Cu) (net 10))
 (segment (start 120.34 80.33) (end 124.04 80.33) (width 0.5) (layer F.Cu) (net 10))
 (segment (start 124.72 79.65) (end 124.72 78.16) (width 0.5) (layer F.Cu) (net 10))
 (segment (start 124.04 80.33) (end 124.72 79.65) (width 0.5) (layer F.Cu) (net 10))
 (segment (start 126.95 62.04) (end 126.52 61.61) (width 0.5) (layer B.Cu) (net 5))
 (segment (start 126.52 60.34) (end 126.6 60.26) (width 0.5) (layer B.Cu) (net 5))
 (segment (start 126.52 61.61) (end 126.52 60.34) (width 0.5) (layer B.Cu) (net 5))
 (segment (start 127.27 62.04) (end 128.8 60.51) (width 0.5) (layer B.Cu) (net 5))
 (segment (start 126.95 62.04) (end 127.27 62.04) (width 0.5) (layer B.Cu) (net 5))
 (segment (start 125.7808 63.0492) (end 126.82 62.01) (width 0.5) (layer B.Cu) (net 5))
 (segment (start 125.7808 64.0842) (end 125.7808 63.0492) (width 0.5) (layer B.Cu) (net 5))
 (segment (start 122.3 60.51) (end 128.8 60.51) (width 0.5) (layer F.Cu) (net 5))
 (segment (start 132.679999 65.520001) (end 130.98 67.22) (width 0.5) (layer B.Cu) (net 16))
 (segment (start 133.485001 65.520001) (end 132.679999 65.520001) (width 0.5) (layer B.Cu) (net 16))
 (segment (start 135.188 63.817002) (end 133.485001 65.520001) (width 0.5) (layer B.Cu) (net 16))
 (segment (start 135.188 60.69) (end 135.188 63.817002) (width 0.5) (layer B.Cu) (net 16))
 (segment (start 130.048 76.832) (end 128.72 78.16) (width 0.5) (layer F.Cu) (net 12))
 (segment (start 130.048 75.3488) (end 130.048 76.832) (width 0.5) (layer F.Cu) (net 12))
 (segment (start 124.72 57.64) (end 124.7 57.66) (width 0.5) (layer B.Cu) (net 3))
 (segment (start 124.72 55.66) (end 124.72 57.64) (width 0.5) (layer B.Cu) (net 3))
 (segment (start 124.7 57.66) (end 124.7 57.66) (width 0.5) (layer B.Cu) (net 3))
 (via (at 124.7 57.66) (size 0.8) (drill 0.4) (layers F.Cu B.Cu) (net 3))
 (segment (start 125.743536 70.83001) (end 126.45 70.123546) (width 0.5) (layer F.Cu) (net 3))
 (segment (start 125.534788 70.83001) (end 125.743536 70.83001) (width 0.5) (layer F.Cu) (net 3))
 (segment (start 124.137601 72.227197) (end 125.534788 70.83001) (width 0.5) (layer F.Cu) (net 3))
 (segment (start 124.137601 76.742399) (end 124.137601 72.227197) (width 0.5) (layer F.Cu) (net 3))
 (segment (start 122.72 78.16) (end 124.137601 76.742399) (width 0.5) (layer F.Cu) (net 3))
 (segment (start 124.7 57.66) (end 124.940001 57.419999) (width 0.5) (layer F.Cu) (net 3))
 (segment (start 132.440001 57.419999) (end 133.98 58.959998) (width 0.5) (layer F.Cu) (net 3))
 (segment (start 124.940001 57.419999) (end 132.440001 57.419999) (width 0.5) (layer F.Cu) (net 3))
 (segment (start 133.98 58.959998) (end 133.98 65.76) (width 0.5) (layer F.Cu) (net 3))
 (segment (start 133.98 65.76) (end 132.2 67.54) (width 0.5) (layer F.Cu) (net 3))
 (segment (start 127.37 67.54) (end 126.45 68.46) (width 0.5) (layer F.Cu) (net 3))
 (segment (start 132.2 67.54) (end 127.37 67.54) (width 0.5) (layer F.Cu) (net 3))
 (segment (start 126.45 70.123546) (end 126.45 68.46) (width 0.5) (layer F.Cu) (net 3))
 (segment (start 123.0376 71.8749) (end 125.0825 69.83) (width 0.5) (layer F.Cu) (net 18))
 (segment (start 123.0376 73.0188) (end 123.0376 71.8749) (width 0.5) (layer F.Cu) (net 18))
 (segment (start 123.0376 75.8424) (end 120.72 78.16) (width 0.5) (layer F.Cu) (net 9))
 (segment (start 123.0376 75.4188) (end 123.0376 75.8424) (width 0.5) (layer F.Cu) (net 9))
 (segment (start 131.41 60.495) (end 131.45 60.535) (width 0.5) (layer F.Cu) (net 19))
 (segment (start 131.41 58.52) (end 131.41 60.495) (width 0.5) (layer F.Cu) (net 19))
 (segment (start 123.13 58.69) (end 124.7 60.26) (width 0.5) (layer B.Cu) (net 4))
 (segment (start 122.88 58.69) (end 123.13 58.69) (width 0.5) (layer B.Cu) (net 4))
 (segment (start 122.88 56.59) (end 122.3 56.01) (width 0.5) (layer B.Cu) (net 4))
 (segment (start 122.88 58.69) (end 122.88 56.59) (width 0.5) (layer B.Cu) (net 4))
 (segment (start 128.8 56.01) (end 122.3 56.01) (width 0.5) (layer F.Cu) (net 4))
 (segment (start 128.91 56.12) (end 128.8 56.01) (width 0.5) (layer F.Cu) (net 4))
 (segment (start 131.41 56.12) (end 128.91 56.12) (width 0.5) (layer F.Cu) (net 4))
 (segment (start 129.59 66.25) (end 130.84 66.25) (width 0.5) (layer F.Cu) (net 17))
 (segment (start 130.84 66.25) (end 132.9 64.19) (width 0.5) (layer F.Cu) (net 17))
 (segment (start 132.9 64.19) (end 132.9 64.19) (width 0.5) (layer F.Cu) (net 17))
 (via (at 132.9 64.19) (size 0.8) (drill 0.4) (layers F.Cu B.Cu) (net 17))
 (segment (start 130.98 61.354) (end 130.98 64.17) (width 0.5) (layer B.Cu) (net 6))
 (segment (start 131.484 60.85) (end 130.98 61.354) (width 0.5) (layer B.Cu) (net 6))
 (segment (start 129.89 63.85) (end 130.96 64.92) (width 0.5) (layer F.Cu) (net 6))
 (segment (start 129.59 63.85) (end 129.89 63.85) (width 0.5) (layer F.Cu) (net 6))
 (segment (start 128.91 64.53) (end 129.59 63.85) (width 0.5) (layer F.Cu) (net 6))
 (segment (start 127.21 64.53) (end 128.91 64.53) (width 0.5) (layer F.Cu) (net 6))
 (segment (start 128.458011 58.170009) (end 125.774996 58.170009) (width 0.5) (layer F.Cu) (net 1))
 (via (at 125.774996 58.170009) (size 0.8) (drill 0.4) (layers F.Cu B.Cu) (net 1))
 (segment (start 125.21 63.58) (end 127.728002 63.58) (width 0.5) (layer F.Cu) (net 1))
 (segment (start 127.728002 63.58) (end 130.150001 61.158001) (width 0.5) (layer F.Cu) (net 1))
 (segment (start 130.150001 61.158001) (end 130.150001 59.861999) (width 0.5) (layer F.Cu) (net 1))
 (segment (start 130.150001 59.861999) (end 128.458011 58.170009) (width 0.5) (layer F.Cu) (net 1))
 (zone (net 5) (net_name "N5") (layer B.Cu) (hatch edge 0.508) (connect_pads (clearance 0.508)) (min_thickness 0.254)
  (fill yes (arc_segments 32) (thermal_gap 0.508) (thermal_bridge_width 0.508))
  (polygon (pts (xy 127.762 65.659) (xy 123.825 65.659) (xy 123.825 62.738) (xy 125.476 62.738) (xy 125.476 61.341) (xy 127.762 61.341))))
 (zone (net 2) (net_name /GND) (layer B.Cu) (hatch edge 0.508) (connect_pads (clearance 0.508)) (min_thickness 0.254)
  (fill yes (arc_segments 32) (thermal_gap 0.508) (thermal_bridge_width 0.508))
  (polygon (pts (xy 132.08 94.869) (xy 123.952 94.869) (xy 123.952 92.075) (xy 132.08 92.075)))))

